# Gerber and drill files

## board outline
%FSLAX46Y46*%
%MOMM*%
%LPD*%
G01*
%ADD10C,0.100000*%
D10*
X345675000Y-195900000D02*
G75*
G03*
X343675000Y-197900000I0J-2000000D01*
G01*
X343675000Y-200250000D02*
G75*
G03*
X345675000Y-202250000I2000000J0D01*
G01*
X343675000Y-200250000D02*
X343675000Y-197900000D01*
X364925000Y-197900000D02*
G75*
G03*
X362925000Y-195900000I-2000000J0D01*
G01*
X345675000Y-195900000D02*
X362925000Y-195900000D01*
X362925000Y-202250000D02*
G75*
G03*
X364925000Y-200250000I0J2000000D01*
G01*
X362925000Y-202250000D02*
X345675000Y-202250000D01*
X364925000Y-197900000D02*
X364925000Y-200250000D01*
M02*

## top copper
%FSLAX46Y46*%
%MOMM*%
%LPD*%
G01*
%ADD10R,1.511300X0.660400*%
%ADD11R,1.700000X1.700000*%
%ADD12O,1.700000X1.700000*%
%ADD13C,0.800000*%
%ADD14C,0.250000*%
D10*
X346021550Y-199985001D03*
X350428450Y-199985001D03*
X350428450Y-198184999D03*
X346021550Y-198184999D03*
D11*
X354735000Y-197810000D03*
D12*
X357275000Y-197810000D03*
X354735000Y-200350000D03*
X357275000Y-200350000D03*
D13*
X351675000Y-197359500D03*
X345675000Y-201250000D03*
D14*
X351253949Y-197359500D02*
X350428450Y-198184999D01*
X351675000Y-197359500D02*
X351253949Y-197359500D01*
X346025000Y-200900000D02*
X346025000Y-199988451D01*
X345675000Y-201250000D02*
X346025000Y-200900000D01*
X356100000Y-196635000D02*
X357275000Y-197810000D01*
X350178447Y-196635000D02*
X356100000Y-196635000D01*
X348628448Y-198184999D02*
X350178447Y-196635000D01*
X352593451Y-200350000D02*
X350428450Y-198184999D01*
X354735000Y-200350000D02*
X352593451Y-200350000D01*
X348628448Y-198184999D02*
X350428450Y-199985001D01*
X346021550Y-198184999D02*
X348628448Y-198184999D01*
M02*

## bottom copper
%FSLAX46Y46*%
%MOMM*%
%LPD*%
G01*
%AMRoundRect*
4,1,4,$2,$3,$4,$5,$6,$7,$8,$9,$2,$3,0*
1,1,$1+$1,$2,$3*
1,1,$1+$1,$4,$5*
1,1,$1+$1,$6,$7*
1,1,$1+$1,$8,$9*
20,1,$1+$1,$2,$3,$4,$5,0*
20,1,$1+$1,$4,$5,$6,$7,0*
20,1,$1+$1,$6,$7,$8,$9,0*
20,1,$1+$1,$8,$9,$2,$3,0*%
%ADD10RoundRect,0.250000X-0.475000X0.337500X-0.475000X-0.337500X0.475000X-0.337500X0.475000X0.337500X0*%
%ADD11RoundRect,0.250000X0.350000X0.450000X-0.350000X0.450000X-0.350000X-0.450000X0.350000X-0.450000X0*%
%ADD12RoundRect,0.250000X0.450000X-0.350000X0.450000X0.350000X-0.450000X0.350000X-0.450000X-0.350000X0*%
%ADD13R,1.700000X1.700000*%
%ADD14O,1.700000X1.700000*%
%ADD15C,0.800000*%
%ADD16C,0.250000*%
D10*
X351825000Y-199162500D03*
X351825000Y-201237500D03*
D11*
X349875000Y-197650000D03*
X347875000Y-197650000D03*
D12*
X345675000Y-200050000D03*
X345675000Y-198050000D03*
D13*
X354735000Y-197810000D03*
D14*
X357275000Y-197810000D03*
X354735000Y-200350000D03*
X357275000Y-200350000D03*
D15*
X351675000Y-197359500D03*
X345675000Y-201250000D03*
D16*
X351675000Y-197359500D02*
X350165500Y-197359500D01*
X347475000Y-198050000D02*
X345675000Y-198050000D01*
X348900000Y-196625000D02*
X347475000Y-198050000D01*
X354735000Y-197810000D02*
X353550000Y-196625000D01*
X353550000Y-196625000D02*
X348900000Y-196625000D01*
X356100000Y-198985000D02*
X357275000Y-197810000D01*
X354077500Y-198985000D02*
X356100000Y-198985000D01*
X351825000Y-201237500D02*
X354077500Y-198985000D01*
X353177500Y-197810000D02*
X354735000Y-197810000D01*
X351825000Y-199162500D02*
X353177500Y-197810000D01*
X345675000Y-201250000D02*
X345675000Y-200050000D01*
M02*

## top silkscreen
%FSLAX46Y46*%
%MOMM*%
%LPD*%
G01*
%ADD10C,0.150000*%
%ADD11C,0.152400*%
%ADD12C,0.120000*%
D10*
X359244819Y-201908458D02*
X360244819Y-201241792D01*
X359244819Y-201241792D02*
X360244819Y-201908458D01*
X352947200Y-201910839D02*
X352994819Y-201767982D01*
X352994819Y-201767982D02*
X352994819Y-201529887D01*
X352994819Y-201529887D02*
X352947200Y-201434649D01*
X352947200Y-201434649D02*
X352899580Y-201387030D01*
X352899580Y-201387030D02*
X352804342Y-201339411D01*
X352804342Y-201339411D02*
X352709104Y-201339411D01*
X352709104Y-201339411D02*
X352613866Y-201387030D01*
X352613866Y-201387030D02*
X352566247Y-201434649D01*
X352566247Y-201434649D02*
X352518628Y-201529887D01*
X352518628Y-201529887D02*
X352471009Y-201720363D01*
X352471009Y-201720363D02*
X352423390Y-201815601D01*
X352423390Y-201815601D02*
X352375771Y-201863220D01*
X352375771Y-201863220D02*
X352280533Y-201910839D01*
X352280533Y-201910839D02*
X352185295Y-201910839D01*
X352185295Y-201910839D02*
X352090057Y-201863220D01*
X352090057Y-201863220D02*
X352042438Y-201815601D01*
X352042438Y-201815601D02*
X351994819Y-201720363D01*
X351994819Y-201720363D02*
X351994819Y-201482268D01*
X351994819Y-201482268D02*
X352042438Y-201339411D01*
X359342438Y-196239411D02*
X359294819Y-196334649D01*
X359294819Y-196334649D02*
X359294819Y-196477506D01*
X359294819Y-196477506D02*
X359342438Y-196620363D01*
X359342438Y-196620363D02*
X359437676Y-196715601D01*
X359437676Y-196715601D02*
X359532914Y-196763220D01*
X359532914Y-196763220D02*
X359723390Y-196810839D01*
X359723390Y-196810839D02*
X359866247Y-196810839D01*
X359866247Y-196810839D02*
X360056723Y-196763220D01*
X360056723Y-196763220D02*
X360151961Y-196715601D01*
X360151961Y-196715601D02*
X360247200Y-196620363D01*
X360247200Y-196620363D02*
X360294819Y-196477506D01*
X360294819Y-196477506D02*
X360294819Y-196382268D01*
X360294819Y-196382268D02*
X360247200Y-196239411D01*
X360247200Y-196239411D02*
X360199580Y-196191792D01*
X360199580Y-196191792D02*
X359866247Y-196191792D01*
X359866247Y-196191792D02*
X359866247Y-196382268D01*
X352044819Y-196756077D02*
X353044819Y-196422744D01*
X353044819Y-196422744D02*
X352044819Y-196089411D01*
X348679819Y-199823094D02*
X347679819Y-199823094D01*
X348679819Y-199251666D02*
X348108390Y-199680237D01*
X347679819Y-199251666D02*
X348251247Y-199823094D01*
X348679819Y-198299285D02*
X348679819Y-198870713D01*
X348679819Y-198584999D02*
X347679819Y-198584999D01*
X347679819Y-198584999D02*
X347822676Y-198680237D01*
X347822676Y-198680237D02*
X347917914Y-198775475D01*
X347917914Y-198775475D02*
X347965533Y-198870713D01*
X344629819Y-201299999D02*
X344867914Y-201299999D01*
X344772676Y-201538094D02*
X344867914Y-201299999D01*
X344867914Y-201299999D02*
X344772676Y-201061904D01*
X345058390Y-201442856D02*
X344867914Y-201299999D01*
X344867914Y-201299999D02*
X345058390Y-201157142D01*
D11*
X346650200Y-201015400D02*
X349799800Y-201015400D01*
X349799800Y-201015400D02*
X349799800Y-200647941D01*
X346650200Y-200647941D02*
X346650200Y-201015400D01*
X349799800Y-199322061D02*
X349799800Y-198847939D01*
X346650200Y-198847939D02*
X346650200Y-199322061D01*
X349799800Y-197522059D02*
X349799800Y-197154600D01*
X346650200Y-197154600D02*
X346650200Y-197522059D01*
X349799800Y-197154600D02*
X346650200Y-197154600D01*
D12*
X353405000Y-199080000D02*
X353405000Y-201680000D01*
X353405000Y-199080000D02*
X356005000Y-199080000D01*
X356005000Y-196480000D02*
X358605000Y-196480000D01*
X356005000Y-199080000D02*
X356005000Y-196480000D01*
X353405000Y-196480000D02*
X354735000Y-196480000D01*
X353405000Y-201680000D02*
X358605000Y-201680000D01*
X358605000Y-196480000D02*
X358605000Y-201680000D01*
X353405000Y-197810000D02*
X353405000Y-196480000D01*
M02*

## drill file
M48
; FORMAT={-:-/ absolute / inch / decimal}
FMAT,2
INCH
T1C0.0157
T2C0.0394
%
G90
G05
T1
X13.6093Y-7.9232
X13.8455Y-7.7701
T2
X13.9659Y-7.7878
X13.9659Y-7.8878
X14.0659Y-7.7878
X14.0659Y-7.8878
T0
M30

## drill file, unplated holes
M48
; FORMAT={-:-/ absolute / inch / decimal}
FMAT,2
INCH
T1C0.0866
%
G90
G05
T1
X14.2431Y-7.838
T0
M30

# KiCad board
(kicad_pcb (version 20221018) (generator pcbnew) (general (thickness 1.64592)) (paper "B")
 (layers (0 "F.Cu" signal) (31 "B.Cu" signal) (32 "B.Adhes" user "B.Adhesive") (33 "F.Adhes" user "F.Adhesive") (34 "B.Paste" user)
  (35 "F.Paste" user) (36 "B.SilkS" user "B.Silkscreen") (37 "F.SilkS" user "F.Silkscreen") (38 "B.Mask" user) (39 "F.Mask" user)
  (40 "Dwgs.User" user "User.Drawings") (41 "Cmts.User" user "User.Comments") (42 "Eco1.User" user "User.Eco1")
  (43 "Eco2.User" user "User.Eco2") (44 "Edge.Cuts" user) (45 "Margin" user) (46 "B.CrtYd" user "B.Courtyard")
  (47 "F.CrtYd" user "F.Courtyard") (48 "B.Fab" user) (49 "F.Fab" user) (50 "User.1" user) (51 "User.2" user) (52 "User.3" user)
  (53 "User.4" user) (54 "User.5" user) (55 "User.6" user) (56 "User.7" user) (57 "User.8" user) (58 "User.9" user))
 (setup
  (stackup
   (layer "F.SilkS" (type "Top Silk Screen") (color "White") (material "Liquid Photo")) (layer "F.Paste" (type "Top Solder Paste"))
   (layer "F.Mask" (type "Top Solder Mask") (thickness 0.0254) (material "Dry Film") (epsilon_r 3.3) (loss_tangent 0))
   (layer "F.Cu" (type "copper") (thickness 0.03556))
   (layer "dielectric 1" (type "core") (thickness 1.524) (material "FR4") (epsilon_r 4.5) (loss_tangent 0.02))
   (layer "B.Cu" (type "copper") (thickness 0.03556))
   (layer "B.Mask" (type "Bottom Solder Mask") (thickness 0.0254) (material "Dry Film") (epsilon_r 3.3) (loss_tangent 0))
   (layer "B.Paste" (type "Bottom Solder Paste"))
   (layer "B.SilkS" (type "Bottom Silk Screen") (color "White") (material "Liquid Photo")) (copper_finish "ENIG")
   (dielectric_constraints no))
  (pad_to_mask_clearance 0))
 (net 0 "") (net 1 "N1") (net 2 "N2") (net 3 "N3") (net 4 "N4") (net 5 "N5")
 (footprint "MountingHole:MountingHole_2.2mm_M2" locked (layer "F.Cu") (at 361.775 199.085)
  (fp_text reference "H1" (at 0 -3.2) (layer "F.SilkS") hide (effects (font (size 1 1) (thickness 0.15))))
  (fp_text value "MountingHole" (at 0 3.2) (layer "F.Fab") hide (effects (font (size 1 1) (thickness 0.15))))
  (pad "" np_thru_hole circle locked (at 0 0) (size 2.2 2.2) (drill 2.2) (layers "*.Cu" "*.Mask")))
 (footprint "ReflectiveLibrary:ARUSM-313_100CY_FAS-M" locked (layer "F.Cu") (at 348.225 199.085 90)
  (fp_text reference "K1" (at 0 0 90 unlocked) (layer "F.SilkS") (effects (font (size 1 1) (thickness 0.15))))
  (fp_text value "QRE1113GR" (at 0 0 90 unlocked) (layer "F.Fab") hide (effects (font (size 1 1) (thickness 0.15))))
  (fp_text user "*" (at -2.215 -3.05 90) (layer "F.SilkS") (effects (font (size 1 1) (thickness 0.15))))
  (fp_line (start -1.9304 -1.5748) (end -1.9304 1.5748) (stroke (width 0.1524) (type solid)) (layer "F.SilkS"))
  (fp_line (start -1.9304 1.5748) (end -1.562941 1.5748) (stroke (width 0.1524) (type solid)) (layer "F.SilkS"))
  (fp_line (start -1.562941 -1.5748) (end -1.9304 -1.5748) (stroke (width 0.1524) (type solid)) (layer "F.SilkS"))
  (fp_line (start -0.237061 1.5748) (end 0.237061 1.5748) (stroke (width 0.1524) (type solid)) (layer "F.SilkS"))
  (fp_line (start 0.237061 -1.5748) (end -0.237061 -1.5748) (stroke (width 0.1524) (type solid)) (layer "F.SilkS"))
  (fp_line (start 1.562941 1.5748) (end 1.9304 1.5748) (stroke (width 0.1524) (type solid)) (layer "F.SilkS"))
  (fp_line (start 1.9304 -1.5748) (end 1.562941 -1.5748) (stroke (width 0.1524) (type solid)) (layer "F.SilkS"))
  (fp_line (start 1.9304 1.5748) (end 1.9304 -1.5748) (stroke (width 0.1524) (type solid)) (layer "F.SilkS"))
  (pad "1" smd rect locked (at -0.900001 -2.20345 90) (size 0.6604 1.5113) (layers "F.Cu" "F.Paste" "F.Mask") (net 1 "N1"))
  (pad "2" smd rect locked (at -0.900001 2.20345 90) (size 0.6604 1.5113) (layers "F.Cu" "F.Paste" "F.Mask") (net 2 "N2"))
  (pad "3" smd rect locked (at 0.900001 2.20345 90) (size 0.6604 1.5113) (layers "F.Cu" "F.Paste" "F.Mask") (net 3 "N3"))
  (pad "4" smd rect locked (at 0.900001 -2.20345 90) (size 0.6604 1.5113) (layers "F.Cu" "F.Paste" "F.Mask") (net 2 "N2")))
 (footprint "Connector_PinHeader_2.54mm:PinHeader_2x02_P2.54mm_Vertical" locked (layer "F.Cu") (at 354.735 197.81)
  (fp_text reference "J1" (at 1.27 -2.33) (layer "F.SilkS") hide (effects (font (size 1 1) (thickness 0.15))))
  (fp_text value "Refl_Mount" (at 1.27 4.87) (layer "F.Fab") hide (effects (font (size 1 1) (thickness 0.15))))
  (fp_line (start -1.33 -1.33) (end 0 -1.33) (stroke (width 0.12) (type solid)) (layer "F.SilkS"))
  (fp_line (start -1.33 0) (end -1.33 -1.33) (stroke (width 0.12) (type solid)) (layer "F.SilkS"))
  (fp_line (start -1.33 1.27) (end -1.33 3.87) (stroke (width 0.12) (type solid)) (layer "F.SilkS"))
  (fp_line (start -1.33 1.27) (end 1.27 1.27) (stroke (width 0.12) (type solid)) (layer "F.SilkS"))
  (fp_line (start -1.33 3.87) (end 3.87 3.87) (stroke (width 0.12) (type solid)) (layer "F.SilkS"))
  (fp_line (start 1.27 -1.33) (end 3.87 -1.33) (stroke (width 0.12) (type solid)) (layer "F.SilkS"))
  (fp_line (start 1.27 1.27) (end 1.27 -1.33) (stroke (width 0.12) (type solid)) (layer "F.SilkS"))
  (fp_line (start 3.87 -1.33) (end 3.87 3.87) (stroke (width 0.12) (type solid)) (layer "F.SilkS"))
  (pad "1" thru_hole rect locked (at 0 0) (size 1.7 1.7) (drill 1) (layers "*.Cu" "*.Mask") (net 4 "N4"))
  (pad "2" thru_hole oval locked (at 2.54 0) (size 1.7 1.7) (drill 1) (layers "*.Cu" "*.Mask") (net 2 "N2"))
  (pad "3" thru_hole oval locked (at 0 2.54) (size 1.7 1.7) (drill 1) (layers "*.Cu" "*.Mask") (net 3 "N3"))
  (pad "4" thru_hole oval locked (at 2.54 2.54) (size 1.7 1.7) (drill 1) (layers "*.Cu" "*.Mask") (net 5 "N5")))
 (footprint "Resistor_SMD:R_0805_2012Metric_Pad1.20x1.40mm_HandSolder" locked (layer "B.Cu") (at 348.875 197.65 180)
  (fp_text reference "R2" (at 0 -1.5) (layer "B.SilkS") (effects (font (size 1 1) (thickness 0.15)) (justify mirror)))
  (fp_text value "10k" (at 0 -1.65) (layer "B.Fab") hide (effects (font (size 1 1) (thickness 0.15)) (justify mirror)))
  (pad "1" smd roundrect locked (at -1 0 180) (size 1.2 1.4) (layers "B.Cu" "B.Paste" "B.Mask") (roundrect_rratio 0.2083333333) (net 3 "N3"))
  (pad "2" smd roundrect locked (at 1 0 180) (size 1.2 1.4) (layers "B.Cu" "B.Paste" "B.Mask") (roundrect_rratio 0.2083333333) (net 4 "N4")))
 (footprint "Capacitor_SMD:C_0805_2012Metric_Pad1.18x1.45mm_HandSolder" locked (layer "B.Cu") (at 351.825 200.2 -90)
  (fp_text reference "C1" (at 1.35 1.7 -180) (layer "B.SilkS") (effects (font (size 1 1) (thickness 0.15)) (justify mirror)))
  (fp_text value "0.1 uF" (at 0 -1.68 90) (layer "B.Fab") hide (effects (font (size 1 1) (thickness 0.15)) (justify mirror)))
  (pad "1" smd roundrect locked (at -1.0375 0 270) (size 1.175 1.45) (layers "B.Cu" "B.Paste" "B.Mask") (roundrect_rratio 0.212766)
   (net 4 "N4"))
  (pad "2" smd roundrect locked (at 1.0375 0 270) (size 1.175 1.45) (layers "B.Cu" "B.Paste" "B.Mask") (roundrect_rratio 0.212766)
   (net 2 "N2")))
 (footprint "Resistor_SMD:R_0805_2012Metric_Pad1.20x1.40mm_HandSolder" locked (layer "B.Cu") (at 345.675 199.05 90)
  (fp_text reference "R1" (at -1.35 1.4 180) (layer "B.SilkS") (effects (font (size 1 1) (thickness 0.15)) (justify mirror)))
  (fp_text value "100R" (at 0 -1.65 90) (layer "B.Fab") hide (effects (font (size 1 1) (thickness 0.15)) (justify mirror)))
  (pad "1" smd roundrect locked (at -1 0 90) (size 1.2 1.4) (layers "B.Cu" "B.Paste" "B.Mask") (roundrect_rratio 0.2083333333) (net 1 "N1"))
  (pad "2" smd roundrect locked (at 1 0 90) (size 1.2 1.4) (layers "B.Cu" "B.Paste" "B.Mask") (roundrect_rratio 0.2083333333) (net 4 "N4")))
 (gr_arc locked (start 362.925 195.9) (mid 364.339214 196.485786) (end 364.925 197.9) (stroke (width 0.1) (type default))
  (layer "Edge.Cuts"))
 (gr_arc locked (start 345.675 202.25) (mid 344.260786 201.664214) (end 343.675 200.25) (stroke (width 0.1) (type default))
  (layer "Edge.Cuts"))
 (gr_line locked (start 345.675 195.9) (end 362.925 195.9) (stroke (width 0.1) (type default)) (layer "Edge.Cuts"))
 (gr_line locked (start 364.925 197.9) (end 364.925 200.25) (stroke (width 0.1) (type default)) (layer "Edge.Cuts"))
 (gr_arc locked (start 343.675 197.9) (mid 344.260786 196.485786) (end 345.675 195.9) (stroke (width 0.1) (type default))
  (layer "Edge.Cuts"))
 (gr_line locked (start 362.925 202.25) (end 345.675 202.25) (stroke (width 0.1) (type default)) (layer "Edge.Cuts"))
 (gr_arc locked (start 364.925 200.25) (mid 364.339214 201.664214) (end 362.925 202.25) (stroke (width 0.1) (type default))
  (layer "Edge.Cuts"))
 (gr_line locked (start 343.675 200.25) (end 343.675 197.9) (stroke (width 0.1) (type default)) (layer "Edge.Cuts"))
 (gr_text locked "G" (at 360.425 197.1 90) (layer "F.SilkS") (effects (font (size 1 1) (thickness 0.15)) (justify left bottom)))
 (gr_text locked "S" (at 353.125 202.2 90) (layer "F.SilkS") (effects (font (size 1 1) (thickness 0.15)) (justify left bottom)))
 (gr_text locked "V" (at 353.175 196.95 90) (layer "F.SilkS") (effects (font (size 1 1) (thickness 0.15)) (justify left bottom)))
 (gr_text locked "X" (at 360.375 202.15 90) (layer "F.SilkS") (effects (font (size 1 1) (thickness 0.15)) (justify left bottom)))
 (segment locked (start 351.825 199.1625) (end 353.1775 197.81) (width 0.25) (layer "B.Cu") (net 4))
 (segment locked (start 353.55 196.625) (end 348.9 196.625) (width 0.25) (layer "B.Cu") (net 4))
 (segment locked (start 347.475 198.05) (end 345.675 198.05) (width 0.25) (layer "B.Cu") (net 4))
 (segment locked (start 353.1775 197.81) (end 354.735 197.81) (width 0.25) (layer "B.Cu") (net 4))
 (segment locked (start 354.735 197.81) (end 353.55 196.625) (width 0.25) (layer "B.Cu") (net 4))
 (segment locked (start 348.9 196.625) (end 347.475 198.05) (width 0.25) (layer "B.Cu") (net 4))
 (segment locked (start 348.628448 198.184999) (end 350.42845 199.985001) (width 0.25) (layer "F.Cu") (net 2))
 (segment locked (start 350.178447 196.635) (end 356.1 196.635) (width 0.25) (layer "F.Cu") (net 2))
 (segment locked (start 348.628448 198.184999) (end 350.178447 196.635) (width 0.25) (layer "F.Cu") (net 2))
 (segment locked (start 346.02155 198.184999) (end 348.628448 198.184999) (width 0.25) (layer "F.Cu") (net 2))
 (segment locked (start 356.1 196.635) (end 357.275 197.81) (width 0.25) (layer "F.Cu") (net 2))
 (segment locked (start 351.825 201.2375) (end 354.0775 198.985) (width 0.25) (layer "B.Cu") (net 2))
 (segment locked (start 354.0775 198.985) (end 356.1 198.985) (width 0.25) (layer "B.Cu") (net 2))
 (segment locked (start 356.1 198.985) (end 357.275 197.81) (width 0.25) (layer "B.Cu") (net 2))
 (segment locked (start 351.675 197.3595) (end 351.253949 197.3595) (width 0.25) (layer "F.Cu") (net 3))
 (segment locked (start 351.253949 197.3595) (end 350.42845 198.184999) (width 0.25) (layer "F.Cu") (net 3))
 (segment locked (start 352.593451 200.35) (end 350.42845 198.184999) (width 0.25) (layer "F.Cu") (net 3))
 (segment locked (start 354.735 200.35) (end 352.593451 200.35) (width 0.25) (layer "F.Cu") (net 3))
 (via locked (at 351.675 197.3595) (size 0.8) (drill 0.4) (layers "F.Cu" "B.Cu") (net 3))
 (segment locked (start 351.675 197.3595) (end 350.1655 197.3595) (width 0.25) (layer "B.Cu") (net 3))
 (segment locked (start 346.025 200.9) (end 346.025 199.988451) (width 0.25) (layer "F.Cu") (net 1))
 (segment locked (start 345.675 201.25) (end 346.025 200.9) (width 0.25) (layer "F.Cu") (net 1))
 (via locked (at 345.675 201.25) (size 0.8) (drill 0.4) (layers "F.Cu" "B.Cu") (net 1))
 (segment locked (start 345.675 201.25) (end 345.675 200.05) (width 0.25) (layer "B.Cu") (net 1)))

